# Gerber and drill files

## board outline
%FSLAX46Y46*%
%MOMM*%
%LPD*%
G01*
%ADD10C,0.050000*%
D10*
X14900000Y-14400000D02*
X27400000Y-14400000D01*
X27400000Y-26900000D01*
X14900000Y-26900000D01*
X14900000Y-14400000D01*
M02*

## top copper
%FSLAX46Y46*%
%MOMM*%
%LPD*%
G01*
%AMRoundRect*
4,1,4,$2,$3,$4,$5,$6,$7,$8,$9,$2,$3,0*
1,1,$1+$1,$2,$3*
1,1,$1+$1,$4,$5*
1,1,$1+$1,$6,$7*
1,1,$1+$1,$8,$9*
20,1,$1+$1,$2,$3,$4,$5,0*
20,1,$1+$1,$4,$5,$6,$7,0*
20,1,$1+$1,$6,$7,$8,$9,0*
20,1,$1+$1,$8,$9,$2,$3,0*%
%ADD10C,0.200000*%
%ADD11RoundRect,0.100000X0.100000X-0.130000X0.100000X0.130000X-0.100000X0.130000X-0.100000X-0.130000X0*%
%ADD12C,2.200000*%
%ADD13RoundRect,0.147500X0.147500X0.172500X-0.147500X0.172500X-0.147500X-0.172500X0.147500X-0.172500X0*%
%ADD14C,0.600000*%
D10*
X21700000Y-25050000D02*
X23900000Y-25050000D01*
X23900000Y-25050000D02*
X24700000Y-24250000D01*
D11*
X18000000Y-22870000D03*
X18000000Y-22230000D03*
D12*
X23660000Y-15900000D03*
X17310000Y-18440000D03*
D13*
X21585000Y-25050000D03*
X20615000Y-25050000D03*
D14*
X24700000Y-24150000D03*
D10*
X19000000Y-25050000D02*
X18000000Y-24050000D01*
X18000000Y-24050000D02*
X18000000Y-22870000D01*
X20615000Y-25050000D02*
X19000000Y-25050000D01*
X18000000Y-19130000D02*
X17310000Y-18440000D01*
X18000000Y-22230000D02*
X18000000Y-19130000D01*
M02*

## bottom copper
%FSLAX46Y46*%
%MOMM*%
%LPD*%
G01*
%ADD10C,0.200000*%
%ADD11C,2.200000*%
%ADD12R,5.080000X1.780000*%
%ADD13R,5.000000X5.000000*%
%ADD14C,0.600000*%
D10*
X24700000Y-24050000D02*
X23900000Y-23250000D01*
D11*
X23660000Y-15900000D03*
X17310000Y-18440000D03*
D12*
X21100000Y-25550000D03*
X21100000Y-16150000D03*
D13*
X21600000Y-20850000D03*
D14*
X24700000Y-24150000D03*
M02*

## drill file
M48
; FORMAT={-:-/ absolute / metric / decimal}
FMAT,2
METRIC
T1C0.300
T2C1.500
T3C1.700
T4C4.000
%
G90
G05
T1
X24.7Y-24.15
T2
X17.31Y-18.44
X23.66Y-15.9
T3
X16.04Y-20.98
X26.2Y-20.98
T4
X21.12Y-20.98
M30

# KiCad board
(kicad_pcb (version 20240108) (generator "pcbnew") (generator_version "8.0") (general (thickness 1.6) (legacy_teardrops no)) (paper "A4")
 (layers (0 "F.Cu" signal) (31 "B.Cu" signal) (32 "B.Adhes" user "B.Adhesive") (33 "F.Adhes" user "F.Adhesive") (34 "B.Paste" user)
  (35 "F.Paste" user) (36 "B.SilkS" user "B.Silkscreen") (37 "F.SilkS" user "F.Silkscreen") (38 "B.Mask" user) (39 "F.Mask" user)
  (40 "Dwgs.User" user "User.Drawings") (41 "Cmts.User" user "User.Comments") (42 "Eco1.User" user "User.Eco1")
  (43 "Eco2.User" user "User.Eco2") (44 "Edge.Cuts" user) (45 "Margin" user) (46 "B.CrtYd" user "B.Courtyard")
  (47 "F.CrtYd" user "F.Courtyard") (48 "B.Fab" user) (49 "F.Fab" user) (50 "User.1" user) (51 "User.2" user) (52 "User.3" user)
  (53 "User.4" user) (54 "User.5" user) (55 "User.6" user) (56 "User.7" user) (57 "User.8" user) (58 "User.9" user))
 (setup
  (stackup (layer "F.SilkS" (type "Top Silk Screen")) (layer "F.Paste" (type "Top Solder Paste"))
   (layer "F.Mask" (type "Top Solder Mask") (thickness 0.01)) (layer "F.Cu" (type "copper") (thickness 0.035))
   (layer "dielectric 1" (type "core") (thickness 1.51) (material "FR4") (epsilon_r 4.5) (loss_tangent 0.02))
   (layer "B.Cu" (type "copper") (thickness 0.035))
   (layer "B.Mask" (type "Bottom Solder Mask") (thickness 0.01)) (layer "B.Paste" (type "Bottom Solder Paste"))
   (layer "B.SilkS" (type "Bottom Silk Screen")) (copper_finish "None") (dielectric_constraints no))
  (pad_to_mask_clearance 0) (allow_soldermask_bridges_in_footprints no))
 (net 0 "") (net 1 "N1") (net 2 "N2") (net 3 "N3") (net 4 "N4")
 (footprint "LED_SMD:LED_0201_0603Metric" (layer "F.Cu") (at 18 22.55 90)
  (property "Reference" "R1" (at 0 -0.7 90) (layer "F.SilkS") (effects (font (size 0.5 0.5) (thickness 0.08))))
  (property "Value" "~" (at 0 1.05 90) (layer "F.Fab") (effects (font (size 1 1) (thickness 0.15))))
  (pad "" smd roundrect (at -0.345 0 90) (size 0.318 0.36) (layers "F.Paste") (roundrect_rratio 0.25))
  (pad "" smd roundrect (at 0.345 0 90) (size 0.318 0.36) (layers "F.Paste") (roundrect_rratio 0.25))
  (pad "1" smd roundrect (at -0.32 0 90) (size 0.46 0.4) (layers "F.Cu" "F.Mask") (roundrect_rratio 0.25) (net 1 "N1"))
  (pad "2" smd roundrect (at 0.32 0 90) (size 0.46 0.4) (layers "F.Cu" "F.Mask") (roundrect_rratio 0.25) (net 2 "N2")))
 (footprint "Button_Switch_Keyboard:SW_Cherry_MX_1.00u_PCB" (layer "F.Cu") (at 23.66 15.9)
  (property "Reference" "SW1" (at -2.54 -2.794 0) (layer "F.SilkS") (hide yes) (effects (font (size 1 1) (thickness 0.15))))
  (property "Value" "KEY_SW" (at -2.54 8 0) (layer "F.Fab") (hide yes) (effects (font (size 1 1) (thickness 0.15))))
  (pad "" np_thru_hole circle (at -7.62 5.08) (size 1.7 1.7) (drill 1.7) (layers "*.Cu" "*.Mask"))
  (pad "" np_thru_hole circle (at -2.54 5.08) (size 4 4) (drill 4) (layers "*.Cu" "*.Mask"))
  (pad "" np_thru_hole circle (at 2.54 5.08) (size 1.7 1.7) (drill 1.7) (layers "*.Cu" "*.Mask"))
  (pad "1" thru_hole circle (at 0 0) (size 2.2 2.2) (drill 1.5) (layers "*.Cu" "*.Mask") (remove_unused_layers no) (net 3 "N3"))
  (pad "2" thru_hole circle (at -6.35 2.54) (size 2.2 2.2) (drill 1.5) (layers "*.Cu" "*.Mask") (remove_unused_layers no) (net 2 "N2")))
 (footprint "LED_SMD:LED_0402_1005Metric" (layer "F.Cu") (at 21.1 25.05 180)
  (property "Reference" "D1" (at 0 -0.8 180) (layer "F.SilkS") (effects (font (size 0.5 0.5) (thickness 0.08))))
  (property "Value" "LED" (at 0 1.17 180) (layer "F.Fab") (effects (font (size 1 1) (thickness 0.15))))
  (pad "1" smd roundrect (at -0.485 0 180) (size 0.59 0.64) (layers "F.Cu" "F.Paste" "F.Mask") (roundrect_rratio 0.25) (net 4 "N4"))
  (pad "2" smd roundrect (at 0.485 0 180) (size 0.59 0.64) (layers "F.Cu" "F.Paste" "F.Mask") (roundrect_rratio 0.25) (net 1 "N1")))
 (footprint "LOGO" (layer "F.Cu") (at 15.4 14.85)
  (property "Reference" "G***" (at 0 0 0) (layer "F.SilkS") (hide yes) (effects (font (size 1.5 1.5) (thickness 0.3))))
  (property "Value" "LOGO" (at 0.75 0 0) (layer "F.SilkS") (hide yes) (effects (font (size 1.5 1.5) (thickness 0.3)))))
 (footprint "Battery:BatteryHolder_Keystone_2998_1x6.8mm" (layer "B.Cu") (at 21.1 20.85 90)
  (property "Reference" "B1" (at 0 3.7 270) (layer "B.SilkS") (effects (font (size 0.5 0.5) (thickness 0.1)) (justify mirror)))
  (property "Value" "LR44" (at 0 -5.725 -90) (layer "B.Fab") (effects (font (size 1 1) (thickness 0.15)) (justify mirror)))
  (pad "1" smd rect (at -4.7 0 90) (size 1.78 5.08) (layers "B.Cu" "B.Paste" "B.Mask"))
  (pad "1" smd rect (at 4.7 0 90) (size 1.78 5.08) (layers "B.Cu" "B.Paste" "B.Mask"))
  (pad "2" smd rect (at 0 0.5 90) (size 5 5) (layers "B.Cu" "B.Paste" "B.Mask")))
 (gr_line (start 21.7 25.05) (end 23.9 25.05) (stroke (width 0.2) (type default)) (layer "F.Cu") (net 4))
 (gr_line (start 23.9 25.05) (end 24.7 24.25) (stroke (width 0.2) (type default)) (layer "F.Cu") (net 4))
 (gr_line (start 24.7 24.05) (end 23.9 23.25) (stroke (width 0.2) (type default)) (layer "B.Cu") (net 4))
 (gr_rect (start 14.9 14.4) (end 27.4 26.9) (stroke (width 0.05) (type default)) (fill none) (layer "Edge.Cuts"))
 (segment (start 19 25.05) (end 18 24.05) (width 0.2) (layer "F.Cu") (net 1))
 (segment (start 18 24.05) (end 18 22.87) (width 0.2) (layer "F.Cu") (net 1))
 (segment (start 20.615 25.05) (end 19 25.05) (width 0.2) (layer "F.Cu") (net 1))
 (segment (start 18 19.13) (end 17.31 18.44) (width 0.2) (layer "F.Cu") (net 2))
 (segment (start 18 22.23) (end 18 19.13) (width 0.2) (layer "F.Cu") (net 2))
 (via (at 24.7 24.15) (size 0.6) (drill 0.3) (layers "F.Cu" "B.Cu") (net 4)))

